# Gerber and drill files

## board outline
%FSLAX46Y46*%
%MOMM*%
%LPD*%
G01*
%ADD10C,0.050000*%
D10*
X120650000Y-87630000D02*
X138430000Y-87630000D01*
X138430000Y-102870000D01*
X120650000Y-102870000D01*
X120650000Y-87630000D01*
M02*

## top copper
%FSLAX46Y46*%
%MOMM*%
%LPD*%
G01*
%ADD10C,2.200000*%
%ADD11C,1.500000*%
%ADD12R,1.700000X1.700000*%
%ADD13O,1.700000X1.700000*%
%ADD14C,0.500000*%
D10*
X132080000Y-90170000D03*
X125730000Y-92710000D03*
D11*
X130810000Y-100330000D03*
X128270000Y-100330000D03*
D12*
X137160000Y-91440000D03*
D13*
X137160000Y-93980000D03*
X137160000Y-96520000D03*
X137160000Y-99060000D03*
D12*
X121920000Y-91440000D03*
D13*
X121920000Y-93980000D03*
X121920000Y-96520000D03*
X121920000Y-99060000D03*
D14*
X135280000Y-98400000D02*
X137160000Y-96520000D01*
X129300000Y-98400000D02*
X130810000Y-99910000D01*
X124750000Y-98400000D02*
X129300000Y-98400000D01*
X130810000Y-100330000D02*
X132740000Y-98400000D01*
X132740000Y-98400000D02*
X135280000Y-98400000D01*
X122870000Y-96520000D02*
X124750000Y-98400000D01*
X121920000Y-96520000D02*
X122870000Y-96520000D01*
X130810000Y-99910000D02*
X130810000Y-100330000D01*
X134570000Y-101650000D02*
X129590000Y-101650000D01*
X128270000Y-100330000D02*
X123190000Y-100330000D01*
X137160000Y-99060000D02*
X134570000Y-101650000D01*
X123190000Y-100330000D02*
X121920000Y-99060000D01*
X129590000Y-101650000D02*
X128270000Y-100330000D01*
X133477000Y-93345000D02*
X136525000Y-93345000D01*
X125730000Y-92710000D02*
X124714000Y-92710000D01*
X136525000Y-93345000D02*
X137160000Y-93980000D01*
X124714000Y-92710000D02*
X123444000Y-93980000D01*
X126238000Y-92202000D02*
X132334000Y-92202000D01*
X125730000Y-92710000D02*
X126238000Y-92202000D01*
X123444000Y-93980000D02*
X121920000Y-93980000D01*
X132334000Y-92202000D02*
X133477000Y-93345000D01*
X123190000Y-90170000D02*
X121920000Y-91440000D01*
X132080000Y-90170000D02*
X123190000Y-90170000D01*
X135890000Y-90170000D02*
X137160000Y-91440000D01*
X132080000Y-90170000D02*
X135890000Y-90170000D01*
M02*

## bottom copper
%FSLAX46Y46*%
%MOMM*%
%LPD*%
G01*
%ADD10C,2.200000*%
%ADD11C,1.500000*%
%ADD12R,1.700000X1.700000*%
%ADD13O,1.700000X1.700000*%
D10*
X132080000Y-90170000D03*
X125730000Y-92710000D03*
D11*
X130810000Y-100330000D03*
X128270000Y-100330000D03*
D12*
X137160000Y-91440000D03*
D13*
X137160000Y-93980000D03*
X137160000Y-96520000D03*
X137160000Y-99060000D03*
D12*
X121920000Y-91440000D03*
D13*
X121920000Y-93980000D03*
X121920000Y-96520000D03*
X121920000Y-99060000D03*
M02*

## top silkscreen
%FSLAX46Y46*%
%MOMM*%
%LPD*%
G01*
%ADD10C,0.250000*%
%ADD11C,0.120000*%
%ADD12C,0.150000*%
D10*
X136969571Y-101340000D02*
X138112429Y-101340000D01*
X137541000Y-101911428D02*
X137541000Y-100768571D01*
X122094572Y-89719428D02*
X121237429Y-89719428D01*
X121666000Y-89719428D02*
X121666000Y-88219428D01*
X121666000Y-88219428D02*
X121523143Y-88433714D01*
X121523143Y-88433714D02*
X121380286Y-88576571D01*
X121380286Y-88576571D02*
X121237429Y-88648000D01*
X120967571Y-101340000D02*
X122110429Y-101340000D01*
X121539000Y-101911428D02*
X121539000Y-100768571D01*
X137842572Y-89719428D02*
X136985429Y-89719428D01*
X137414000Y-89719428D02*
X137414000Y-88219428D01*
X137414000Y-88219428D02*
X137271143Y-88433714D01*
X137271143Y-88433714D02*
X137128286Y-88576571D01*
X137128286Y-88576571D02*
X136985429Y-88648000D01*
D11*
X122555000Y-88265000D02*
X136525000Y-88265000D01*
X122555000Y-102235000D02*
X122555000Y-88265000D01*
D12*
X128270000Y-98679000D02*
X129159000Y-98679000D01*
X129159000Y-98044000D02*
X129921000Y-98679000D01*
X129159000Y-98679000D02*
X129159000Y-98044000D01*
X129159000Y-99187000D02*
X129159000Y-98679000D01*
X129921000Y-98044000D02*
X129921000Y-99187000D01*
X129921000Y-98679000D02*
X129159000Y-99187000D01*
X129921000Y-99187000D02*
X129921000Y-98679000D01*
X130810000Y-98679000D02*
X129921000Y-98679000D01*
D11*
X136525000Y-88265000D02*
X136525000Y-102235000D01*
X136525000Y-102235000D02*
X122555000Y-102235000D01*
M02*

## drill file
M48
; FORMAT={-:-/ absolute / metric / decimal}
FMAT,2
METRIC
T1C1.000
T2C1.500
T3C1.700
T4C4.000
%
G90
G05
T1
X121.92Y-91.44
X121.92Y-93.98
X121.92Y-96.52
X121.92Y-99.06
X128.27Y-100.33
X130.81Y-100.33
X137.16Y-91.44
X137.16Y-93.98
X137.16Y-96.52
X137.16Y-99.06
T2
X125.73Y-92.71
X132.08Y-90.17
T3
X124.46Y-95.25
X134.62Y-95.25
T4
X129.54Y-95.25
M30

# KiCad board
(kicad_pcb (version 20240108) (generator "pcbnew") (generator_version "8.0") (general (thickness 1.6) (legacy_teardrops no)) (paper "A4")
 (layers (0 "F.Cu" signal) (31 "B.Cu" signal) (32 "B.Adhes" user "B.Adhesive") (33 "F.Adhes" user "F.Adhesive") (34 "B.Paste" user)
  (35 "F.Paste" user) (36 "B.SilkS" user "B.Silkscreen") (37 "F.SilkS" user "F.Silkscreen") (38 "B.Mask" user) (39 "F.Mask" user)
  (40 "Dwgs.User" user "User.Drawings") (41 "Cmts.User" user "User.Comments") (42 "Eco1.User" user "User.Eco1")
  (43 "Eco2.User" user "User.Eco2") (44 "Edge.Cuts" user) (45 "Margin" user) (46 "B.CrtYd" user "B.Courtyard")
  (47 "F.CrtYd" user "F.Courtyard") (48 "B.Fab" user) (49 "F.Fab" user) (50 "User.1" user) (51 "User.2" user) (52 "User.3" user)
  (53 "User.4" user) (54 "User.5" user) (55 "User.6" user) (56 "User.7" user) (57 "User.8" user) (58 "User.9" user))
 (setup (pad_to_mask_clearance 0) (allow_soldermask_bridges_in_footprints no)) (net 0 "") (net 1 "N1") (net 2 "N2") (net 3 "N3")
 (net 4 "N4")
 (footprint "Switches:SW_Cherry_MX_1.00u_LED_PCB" (layer "F.Cu") (at 132.08 90.17)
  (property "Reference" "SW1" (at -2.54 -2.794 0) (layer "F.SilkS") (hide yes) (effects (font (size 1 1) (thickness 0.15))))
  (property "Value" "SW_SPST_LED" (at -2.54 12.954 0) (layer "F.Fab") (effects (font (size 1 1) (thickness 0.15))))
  (fp_line (start -9.525 -1.905) (end 4.445 -1.905) (stroke (width 0.12) (type solid)) (layer "F.SilkS"))
  (fp_line (start -9.525 12.065) (end -9.525 -1.905) (stroke (width 0.12) (type solid)) (layer "F.SilkS"))
  (fp_line (start -3.81 8.509) (end -2.921 8.509) (stroke (width 0.15) (type default)) (layer "F.SilkS"))
  (fp_line (start -2.921 7.874) (end -2.159 8.509) (stroke (width 0.15) (type default)) (layer "F.SilkS"))
  (fp_line (start -2.921 8.509) (end -2.921 7.874) (stroke (width 0.15) (type default)) (layer "F.SilkS"))
  (fp_line (start -2.921 9.017) (end -2.921 8.509) (stroke (width 0.15) (type default)) (layer "F.SilkS"))
  (fp_line (start -2.159 7.874) (end -2.159 9.017) (stroke (width 0.15) (type default)) (layer "F.SilkS"))
  (fp_line (start -2.159 8.509) (end -2.921 9.017) (stroke (width 0.15) (type default)) (layer "F.SilkS"))
  (fp_line (start -2.159 9.017) (end -2.159 8.509) (stroke (width 0.15) (type default)) (layer "F.SilkS"))
  (fp_line (start -1.27 8.509) (end -2.159 8.509) (stroke (width 0.15) (type default)) (layer "F.SilkS"))
  (fp_line (start 4.445 -1.905) (end 4.445 12.065) (stroke (width 0.12) (type solid)) (layer "F.SilkS"))
  (fp_line (start 4.445 12.065) (end -9.525 12.065) (stroke (width 0.12) (type solid)) (layer "F.SilkS"))
  (pad "" np_thru_hole circle (at -7.62 5.08) (size 1.7 1.7) (drill 1.7) (layers "*.Cu" "*.Mask"))
  (pad "" np_thru_hole circle (at -2.54 5.08) (size 4 4) (drill 4) (layers "*.Cu" "*.Mask"))
  (pad "" np_thru_hole circle (at 2.54 5.08) (size 1.7 1.7) (drill 1.7) (layers "*.Cu" "*.Mask"))
  (pad "1" thru_hole circle (at 0 0) (size 2.2 2.2) (drill 1.5) (layers "*.Cu" "*.Mask") (remove_unused_layers no) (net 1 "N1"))
  (pad "2" thru_hole circle (at -6.35 2.54) (size 2.2 2.2) (drill 1.5) (layers "*.Cu" "*.Mask") (remove_unused_layers no) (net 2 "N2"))
  (pad "3" thru_hole circle (at -1.27 10.16) (size 1.5 1.5) (drill 1) (layers "*.Cu" "*.Mask") (remove_unused_layers no) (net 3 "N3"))
  (pad "4" thru_hole circle (at -3.81 10.16) (size 1.5 1.5) (drill 1) (layers "*.Cu" "*.Mask") (remove_unused_layers no) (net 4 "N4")))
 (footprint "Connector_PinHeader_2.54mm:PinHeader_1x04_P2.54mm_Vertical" (layer "B.Cu") (at 137.16 91.44 180)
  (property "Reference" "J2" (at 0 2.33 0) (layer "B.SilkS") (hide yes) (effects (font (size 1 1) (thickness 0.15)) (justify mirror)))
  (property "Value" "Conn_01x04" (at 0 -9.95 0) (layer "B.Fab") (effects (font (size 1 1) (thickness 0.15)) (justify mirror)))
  (pad "1" thru_hole rect (at 0 0 180) (size 1.7 1.7) (drill 1) (layers "*.Cu" "*.Mask") (remove_unused_layers no) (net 1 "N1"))
  (pad "2" thru_hole oval (at 0 -2.54 180) (size 1.7 1.7) (drill 1) (layers "*.Cu" "*.Mask") (remove_unused_layers no) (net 2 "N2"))
  (pad "3" thru_hole oval (at 0 -5.08 180) (size 1.7 1.7) (drill 1) (layers "*.Cu" "*.Mask") (remove_unused_layers no) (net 3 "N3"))
  (pad "4" thru_hole oval (at 0 -7.62 180) (size 1.7 1.7) (drill 1) (layers "*.Cu" "*.Mask") (remove_unused_layers no) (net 4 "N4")))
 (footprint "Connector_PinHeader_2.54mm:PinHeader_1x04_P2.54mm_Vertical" (layer "B.Cu") (at 121.92 91.44 180)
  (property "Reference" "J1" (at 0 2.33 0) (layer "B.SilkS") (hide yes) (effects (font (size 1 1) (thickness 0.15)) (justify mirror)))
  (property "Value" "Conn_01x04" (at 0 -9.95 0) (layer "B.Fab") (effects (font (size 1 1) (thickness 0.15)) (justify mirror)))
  (pad "1" thru_hole rect (at 0 0 180) (size 1.7 1.7) (drill 1) (layers "*.Cu" "*.Mask") (remove_unused_layers no) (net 1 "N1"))
  (pad "2" thru_hole oval (at 0 -2.54 180) (size 1.7 1.7) (drill 1) (layers "*.Cu" "*.Mask") (remove_unused_layers no) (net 2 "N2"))
  (pad "3" thru_hole oval (at 0 -5.08 180) (size 1.7 1.7) (drill 1) (layers "*.Cu" "*.Mask") (remove_unused_layers no) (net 3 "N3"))
  (pad "4" thru_hole oval (at 0 -7.62 180) (size 1.7 1.7) (drill 1) (layers "*.Cu" "*.Mask") (remove_unused_layers no) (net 4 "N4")))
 (gr_rect (start 120.65 87.63) (end 138.43 102.87) (stroke (width 0.05) (type default)) (fill none) (layer "Edge.Cuts"))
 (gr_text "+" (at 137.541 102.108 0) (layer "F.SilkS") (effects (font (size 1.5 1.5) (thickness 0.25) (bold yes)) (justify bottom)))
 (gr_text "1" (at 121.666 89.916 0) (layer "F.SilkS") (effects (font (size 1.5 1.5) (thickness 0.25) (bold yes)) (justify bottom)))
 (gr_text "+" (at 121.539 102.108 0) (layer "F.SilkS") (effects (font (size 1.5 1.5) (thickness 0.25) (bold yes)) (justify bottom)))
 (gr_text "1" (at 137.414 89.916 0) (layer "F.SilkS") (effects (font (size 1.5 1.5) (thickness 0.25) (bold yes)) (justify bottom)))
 (segment (start 135.28 98.4) (end 137.16 96.52) (width 0.5) (layer "F.Cu") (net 3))
 (segment (start 129.3 98.4) (end 130.81 99.91) (width 0.5) (layer "F.Cu") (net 3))
 (segment (start 124.75 98.4) (end 129.3 98.4) (width 0.5) (layer "F.Cu") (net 3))
 (segment (start 130.81 100.33) (end 132.74 98.4) (width 0.5) (layer "F.Cu") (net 3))
 (segment (start 132.74 98.4) (end 135.28 98.4) (width 0.5) (layer "F.Cu") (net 3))
 (segment (start 122.87 96.52) (end 124.75 98.4) (width 0.5) (layer "F.Cu") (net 3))
 (segment (start 121.92 96.52) (end 122.87 96.52) (width 0.5) (layer "F.Cu") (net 3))
 (segment (start 130.81 99.91) (end 130.81 100.33) (width 0.5) (layer "F.Cu") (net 3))
 (segment (start 134.57 101.65) (end 129.59 101.65) (width 0.5) (layer "F.Cu") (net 4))
 (segment (start 128.27 100.33) (end 123.19 100.33) (width 0.5) (layer "F.Cu") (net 4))
 (segment (start 137.16 99.06) (end 134.57 101.65) (width 0.5) (layer "F.Cu") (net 4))
 (segment (start 123.19 100.33) (end 121.92 99.06) (width 0.5) (layer "F.Cu") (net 4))
 (segment (start 129.59 101.65) (end 128.27 100.33) (width 0.5) (layer "F.Cu") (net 4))
 (segment (start 133.477 93.345) (end 136.525 93.345) (width 0.5) (layer "F.Cu") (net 2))
 (segment (start 125.73 92.71) (end 124.714 92.71) (width 0.5) (layer "F.Cu") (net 2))
 (segment (start 136.525 93.345) (end 137.16 93.98) (width 0.5) (layer "F.Cu") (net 2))
 (segment (start 124.714 92.71) (end 123.444 93.98) (width 0.5) (layer "F.Cu") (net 2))
 (segment (start 126.238 92.202) (end 132.334 92.202) (width 0.5) (layer "F.Cu") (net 2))
 (segment (start 125.73 92.71) (end 126.238 92.202) (width 0.5) (layer "F.Cu") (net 2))
 (segment (start 123.444 93.98) (end 121.92 93.98) (width 0.5) (layer "F.Cu") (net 2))
 (segment (start 132.334 92.202) (end 133.477 93.345) (width 0.5) (layer "F.Cu") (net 2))
 (segment (start 123.19 90.17) (end 121.92 91.44) (width 0.5) (layer "F.Cu") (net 1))
 (segment (start 132.08 90.17) (end 123.19 90.17) (width 0.5) (layer "F.Cu") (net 1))
 (segment (start 135.89 90.17) (end 137.16 91.44) (width 0.5) (layer "F.Cu") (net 1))
 (segment (start 132.08 90.17) (end 135.89 90.17) (width 0.5) (layer "F.Cu") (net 1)))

